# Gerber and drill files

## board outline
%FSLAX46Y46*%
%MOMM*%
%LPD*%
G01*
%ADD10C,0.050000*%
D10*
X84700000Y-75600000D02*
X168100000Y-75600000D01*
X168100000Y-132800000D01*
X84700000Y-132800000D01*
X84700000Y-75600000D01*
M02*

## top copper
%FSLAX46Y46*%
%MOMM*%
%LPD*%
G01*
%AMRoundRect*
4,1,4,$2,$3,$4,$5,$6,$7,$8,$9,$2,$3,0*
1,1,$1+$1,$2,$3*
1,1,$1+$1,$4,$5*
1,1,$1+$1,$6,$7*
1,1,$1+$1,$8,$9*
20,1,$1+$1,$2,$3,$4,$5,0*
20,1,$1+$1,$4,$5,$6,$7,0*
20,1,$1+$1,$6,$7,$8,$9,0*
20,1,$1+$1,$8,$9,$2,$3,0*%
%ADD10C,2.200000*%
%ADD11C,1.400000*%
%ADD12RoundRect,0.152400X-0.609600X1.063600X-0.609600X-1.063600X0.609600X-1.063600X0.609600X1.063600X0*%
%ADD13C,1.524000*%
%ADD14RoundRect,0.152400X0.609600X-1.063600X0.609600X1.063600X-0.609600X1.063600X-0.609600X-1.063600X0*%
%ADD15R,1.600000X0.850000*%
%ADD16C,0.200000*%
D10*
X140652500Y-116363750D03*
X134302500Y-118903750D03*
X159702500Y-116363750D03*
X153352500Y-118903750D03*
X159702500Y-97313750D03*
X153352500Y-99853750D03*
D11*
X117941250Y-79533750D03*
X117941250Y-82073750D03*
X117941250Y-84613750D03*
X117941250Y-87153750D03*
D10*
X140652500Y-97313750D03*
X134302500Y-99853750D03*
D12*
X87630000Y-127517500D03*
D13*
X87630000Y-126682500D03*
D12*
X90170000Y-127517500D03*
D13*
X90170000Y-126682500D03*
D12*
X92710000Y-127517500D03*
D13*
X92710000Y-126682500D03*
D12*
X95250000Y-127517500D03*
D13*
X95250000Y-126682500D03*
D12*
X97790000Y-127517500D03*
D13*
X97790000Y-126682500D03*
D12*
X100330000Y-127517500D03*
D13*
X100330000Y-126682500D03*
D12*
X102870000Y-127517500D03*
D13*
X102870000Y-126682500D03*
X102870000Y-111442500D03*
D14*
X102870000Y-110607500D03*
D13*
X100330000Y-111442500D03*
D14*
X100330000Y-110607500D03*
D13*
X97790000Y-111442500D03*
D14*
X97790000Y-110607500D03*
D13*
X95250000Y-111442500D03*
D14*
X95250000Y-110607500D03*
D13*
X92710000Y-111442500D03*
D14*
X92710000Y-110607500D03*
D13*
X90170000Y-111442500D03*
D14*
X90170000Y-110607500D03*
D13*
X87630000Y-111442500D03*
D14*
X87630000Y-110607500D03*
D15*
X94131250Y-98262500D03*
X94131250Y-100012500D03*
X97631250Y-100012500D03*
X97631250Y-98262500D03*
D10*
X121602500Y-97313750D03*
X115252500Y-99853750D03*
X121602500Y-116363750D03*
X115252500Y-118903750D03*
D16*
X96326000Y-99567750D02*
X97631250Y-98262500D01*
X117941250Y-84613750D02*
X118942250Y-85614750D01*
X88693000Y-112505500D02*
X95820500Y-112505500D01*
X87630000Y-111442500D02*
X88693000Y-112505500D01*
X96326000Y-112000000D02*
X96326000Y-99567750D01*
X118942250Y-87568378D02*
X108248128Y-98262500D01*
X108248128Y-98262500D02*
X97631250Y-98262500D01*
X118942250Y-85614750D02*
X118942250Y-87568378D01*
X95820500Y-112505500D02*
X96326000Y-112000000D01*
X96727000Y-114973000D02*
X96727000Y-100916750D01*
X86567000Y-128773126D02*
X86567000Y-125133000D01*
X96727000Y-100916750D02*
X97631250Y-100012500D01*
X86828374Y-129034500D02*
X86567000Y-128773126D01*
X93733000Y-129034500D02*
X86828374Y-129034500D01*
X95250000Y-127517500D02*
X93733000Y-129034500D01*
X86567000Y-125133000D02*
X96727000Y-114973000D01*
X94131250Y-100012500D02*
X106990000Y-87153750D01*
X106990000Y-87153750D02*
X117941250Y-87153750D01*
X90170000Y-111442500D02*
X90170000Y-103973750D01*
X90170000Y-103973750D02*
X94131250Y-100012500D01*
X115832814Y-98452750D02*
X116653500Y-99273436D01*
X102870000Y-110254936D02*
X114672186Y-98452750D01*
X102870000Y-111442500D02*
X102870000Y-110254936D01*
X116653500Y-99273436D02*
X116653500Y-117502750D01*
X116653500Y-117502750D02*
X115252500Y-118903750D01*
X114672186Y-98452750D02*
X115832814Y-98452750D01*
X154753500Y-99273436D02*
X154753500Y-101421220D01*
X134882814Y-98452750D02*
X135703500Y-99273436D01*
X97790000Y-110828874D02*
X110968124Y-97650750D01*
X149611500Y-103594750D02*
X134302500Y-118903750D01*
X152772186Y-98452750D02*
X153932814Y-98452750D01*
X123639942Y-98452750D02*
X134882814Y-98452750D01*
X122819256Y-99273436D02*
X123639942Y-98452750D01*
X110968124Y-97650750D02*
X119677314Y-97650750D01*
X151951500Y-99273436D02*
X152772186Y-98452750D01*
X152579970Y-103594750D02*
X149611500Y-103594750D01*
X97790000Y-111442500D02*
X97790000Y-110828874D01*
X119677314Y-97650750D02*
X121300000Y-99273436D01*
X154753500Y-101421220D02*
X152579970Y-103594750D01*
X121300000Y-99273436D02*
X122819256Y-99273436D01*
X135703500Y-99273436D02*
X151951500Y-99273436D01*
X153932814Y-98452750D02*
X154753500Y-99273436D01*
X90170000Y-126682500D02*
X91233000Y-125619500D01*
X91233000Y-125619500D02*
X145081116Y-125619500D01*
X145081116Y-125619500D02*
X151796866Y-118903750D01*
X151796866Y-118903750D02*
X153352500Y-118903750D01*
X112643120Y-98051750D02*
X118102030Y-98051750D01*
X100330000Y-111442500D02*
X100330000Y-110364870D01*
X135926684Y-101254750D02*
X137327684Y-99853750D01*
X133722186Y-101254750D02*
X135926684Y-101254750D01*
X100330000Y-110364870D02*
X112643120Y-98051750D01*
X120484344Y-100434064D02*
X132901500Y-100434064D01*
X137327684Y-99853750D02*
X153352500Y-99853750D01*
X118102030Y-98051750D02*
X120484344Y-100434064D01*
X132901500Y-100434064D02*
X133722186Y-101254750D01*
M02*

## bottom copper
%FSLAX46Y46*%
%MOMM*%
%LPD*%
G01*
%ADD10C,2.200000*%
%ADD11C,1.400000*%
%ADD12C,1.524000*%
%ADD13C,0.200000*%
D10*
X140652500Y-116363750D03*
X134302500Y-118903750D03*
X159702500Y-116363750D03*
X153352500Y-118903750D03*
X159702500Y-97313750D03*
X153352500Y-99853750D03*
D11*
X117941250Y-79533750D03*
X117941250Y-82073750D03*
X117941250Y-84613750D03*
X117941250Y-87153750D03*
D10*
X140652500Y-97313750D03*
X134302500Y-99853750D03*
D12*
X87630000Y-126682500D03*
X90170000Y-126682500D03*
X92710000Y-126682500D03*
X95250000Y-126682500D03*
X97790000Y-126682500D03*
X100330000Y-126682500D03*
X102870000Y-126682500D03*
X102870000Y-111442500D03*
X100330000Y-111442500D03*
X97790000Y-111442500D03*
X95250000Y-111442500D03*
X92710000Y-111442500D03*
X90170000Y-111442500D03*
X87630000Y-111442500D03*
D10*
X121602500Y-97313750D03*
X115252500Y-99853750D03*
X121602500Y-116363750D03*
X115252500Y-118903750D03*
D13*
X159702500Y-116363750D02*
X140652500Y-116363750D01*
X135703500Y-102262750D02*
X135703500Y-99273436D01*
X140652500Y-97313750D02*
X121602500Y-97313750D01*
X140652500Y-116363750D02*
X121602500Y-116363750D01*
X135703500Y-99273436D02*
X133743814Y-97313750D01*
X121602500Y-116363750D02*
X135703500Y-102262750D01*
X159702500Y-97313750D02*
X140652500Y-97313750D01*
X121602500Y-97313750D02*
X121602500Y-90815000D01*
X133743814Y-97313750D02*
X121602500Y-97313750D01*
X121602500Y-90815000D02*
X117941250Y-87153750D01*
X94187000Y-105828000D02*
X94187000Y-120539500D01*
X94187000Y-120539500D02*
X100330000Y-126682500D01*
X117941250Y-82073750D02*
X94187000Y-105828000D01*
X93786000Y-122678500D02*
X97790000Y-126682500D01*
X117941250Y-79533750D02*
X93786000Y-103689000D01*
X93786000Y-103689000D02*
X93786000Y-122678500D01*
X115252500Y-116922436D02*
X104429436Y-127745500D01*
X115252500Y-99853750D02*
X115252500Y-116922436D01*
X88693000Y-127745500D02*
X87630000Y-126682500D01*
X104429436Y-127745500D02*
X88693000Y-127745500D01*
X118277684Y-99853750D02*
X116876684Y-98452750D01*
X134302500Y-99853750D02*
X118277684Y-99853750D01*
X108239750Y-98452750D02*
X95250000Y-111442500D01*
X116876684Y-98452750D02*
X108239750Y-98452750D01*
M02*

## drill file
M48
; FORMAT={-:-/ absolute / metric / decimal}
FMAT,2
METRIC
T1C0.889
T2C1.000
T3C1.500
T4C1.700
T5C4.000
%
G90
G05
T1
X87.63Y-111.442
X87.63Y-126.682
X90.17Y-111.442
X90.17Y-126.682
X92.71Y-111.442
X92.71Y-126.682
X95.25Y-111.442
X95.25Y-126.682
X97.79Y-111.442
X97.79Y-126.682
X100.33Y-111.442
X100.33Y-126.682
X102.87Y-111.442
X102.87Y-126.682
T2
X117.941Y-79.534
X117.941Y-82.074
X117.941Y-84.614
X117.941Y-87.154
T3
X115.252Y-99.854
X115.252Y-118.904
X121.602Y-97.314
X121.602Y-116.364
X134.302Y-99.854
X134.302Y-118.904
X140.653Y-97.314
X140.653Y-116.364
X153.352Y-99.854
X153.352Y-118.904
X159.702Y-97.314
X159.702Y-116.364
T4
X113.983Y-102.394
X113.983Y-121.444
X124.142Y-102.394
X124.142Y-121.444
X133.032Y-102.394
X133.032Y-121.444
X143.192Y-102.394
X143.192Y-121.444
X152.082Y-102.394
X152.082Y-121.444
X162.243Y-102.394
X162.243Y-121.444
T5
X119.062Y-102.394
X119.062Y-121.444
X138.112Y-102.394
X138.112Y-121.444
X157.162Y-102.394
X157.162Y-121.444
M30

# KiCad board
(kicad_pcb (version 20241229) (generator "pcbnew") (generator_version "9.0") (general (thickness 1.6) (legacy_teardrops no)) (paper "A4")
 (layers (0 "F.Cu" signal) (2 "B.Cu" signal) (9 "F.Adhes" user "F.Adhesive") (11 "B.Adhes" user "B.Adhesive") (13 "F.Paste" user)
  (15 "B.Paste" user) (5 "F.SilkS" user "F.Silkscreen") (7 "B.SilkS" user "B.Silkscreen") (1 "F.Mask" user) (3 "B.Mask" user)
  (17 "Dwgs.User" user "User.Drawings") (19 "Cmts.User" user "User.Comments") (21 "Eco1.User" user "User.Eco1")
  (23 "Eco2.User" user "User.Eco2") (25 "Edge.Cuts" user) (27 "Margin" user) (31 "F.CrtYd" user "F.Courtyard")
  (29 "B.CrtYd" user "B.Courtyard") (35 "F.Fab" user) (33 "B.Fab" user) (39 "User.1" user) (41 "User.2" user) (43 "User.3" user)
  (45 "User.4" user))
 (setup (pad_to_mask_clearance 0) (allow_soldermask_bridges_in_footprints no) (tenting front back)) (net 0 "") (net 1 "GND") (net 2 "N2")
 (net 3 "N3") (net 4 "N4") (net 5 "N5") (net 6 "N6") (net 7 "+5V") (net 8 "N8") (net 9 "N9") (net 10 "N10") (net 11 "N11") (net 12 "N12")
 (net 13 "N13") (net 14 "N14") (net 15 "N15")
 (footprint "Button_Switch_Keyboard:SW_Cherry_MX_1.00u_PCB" (layer "F.Cu") (at 140.6525 116.36375)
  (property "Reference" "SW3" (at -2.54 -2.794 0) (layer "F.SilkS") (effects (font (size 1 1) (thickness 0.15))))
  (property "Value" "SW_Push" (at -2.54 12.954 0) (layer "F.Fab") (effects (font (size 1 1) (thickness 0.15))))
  (pad "" np_thru_hole circle (at -7.62 5.08) (size 1.7 1.7) (drill 1.7) (layers "*.Cu" "*.Mask"))
  (pad "" np_thru_hole circle (at -2.54 5.08) (size 4 4) (drill 4) (layers "*.Cu" "*.Mask"))
  (pad "" np_thru_hole circle (at 2.54 5.08) (size 1.7 1.7) (drill 1.7) (layers "*.Cu" "*.Mask"))
  (pad "1" thru_hole circle (at 0 0) (size 2.2 2.2) (drill 1.5) (layers "*.Cu" "*.Mask") (remove_unused_layers no) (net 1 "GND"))
  (pad "2" thru_hole circle (at -6.35 2.54) (size 2.2 2.2) (drill 1.5) (layers "*.Cu" "*.Mask") (remove_unused_layers no) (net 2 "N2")))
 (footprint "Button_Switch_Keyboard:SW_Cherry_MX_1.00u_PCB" (layer "F.Cu") (at 159.7025 116.36375)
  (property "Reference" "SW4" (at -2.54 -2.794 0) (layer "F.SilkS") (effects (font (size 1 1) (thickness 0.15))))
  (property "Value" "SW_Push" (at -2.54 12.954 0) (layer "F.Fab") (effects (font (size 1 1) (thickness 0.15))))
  (pad "" np_thru_hole circle (at -7.62 5.08) (size 1.7 1.7) (drill 1.7) (layers "*.Cu" "*.Mask"))
  (pad "" np_thru_hole circle (at -2.54 5.08) (size 4 4) (drill 4) (layers "*.Cu" "*.Mask"))
  (pad "" np_thru_hole circle (at 2.54 5.08) (size 1.7 1.7) (drill 1.7) (layers "*.Cu" "*.Mask"))
  (pad "1" thru_hole circle (at 0 0) (size 2.2 2.2) (drill 1.5) (layers "*.Cu" "*.Mask") (remove_unused_layers no) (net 1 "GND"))
  (pad "2" thru_hole circle (at -6.35 2.54) (size 2.2 2.2) (drill 1.5) (layers "*.Cu" "*.Mask") (remove_unused_layers no) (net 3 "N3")))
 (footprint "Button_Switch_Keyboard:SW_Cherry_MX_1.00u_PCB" (layer "F.Cu") (at 159.7025 97.31375)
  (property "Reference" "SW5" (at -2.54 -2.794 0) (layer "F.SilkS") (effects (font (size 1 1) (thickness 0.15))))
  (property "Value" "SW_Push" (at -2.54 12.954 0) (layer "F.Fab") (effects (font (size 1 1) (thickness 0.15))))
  (pad "" np_thru_hole circle (at -7.62 5.08) (size 1.7 1.7) (drill 1.7) (layers "*.Cu" "*.Mask"))
  (pad "" np_thru_hole circle (at -2.54 5.08) (size 4 4) (drill 4) (layers "*.Cu" "*.Mask"))
  (pad "" np_thru_hole circle (at 2.54 5.08) (size 1.7 1.7) (drill 1.7) (layers "*.Cu" "*.Mask"))
  (pad "1" thru_hole circle (at 0 0) (size 2.2 2.2) (drill 1.5) (layers "*.Cu" "*.Mask") (remove_unused_layers no) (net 1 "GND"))
  (pad "2" thru_hole circle (at -6.35 2.54) (size 2.2 2.2) (drill 1.5) (layers "*.Cu" "*.Mask") (remove_unused_layers no) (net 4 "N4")))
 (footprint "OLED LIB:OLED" (layer "F.Cu") (at 117.94125 83.34375 -90)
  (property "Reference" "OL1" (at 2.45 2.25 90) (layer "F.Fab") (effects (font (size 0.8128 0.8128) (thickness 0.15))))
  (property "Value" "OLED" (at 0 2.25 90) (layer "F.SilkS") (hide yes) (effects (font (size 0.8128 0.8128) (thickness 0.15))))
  (pad "1" thru_hole circle (at -3.81 0 270) (size 1.4 1.4) (drill 1) (layers "*.Cu" "*.Mask") (remove_unused_layers no) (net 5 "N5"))
  (pad "2" thru_hole circle (at -1.27 0 270) (size 1.4 1.4) (drill 1) (layers "*.Cu" "*.Mask") (remove_unused_layers no) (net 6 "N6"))
  (pad "3" thru_hole circle (at 1.27 0 270) (size 1.4 1.4) (drill 1) (layers "*.Cu" "*.Mask") (remove_unused_layers no) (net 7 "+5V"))
  (pad "4" thru_hole circle (at 3.81 0 270) (size 1.4 1.4) (drill 1) (layers "*.Cu" "*.Mask") (remove_unused_layers no) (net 1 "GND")))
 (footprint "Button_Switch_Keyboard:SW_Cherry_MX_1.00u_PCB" (layer "F.Cu") (at 140.6525 97.31375)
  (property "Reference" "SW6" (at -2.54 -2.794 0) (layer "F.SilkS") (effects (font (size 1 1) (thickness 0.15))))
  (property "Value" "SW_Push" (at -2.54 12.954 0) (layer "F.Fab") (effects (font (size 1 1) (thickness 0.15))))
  (pad "" np_thru_hole circle (at -7.62 5.08) (size 1.7 1.7) (drill 1.7) (layers "*.Cu" "*.Mask"))
  (pad "" np_thru_hole circle (at -2.54 5.08) (size 4 4) (drill 4) (layers "*.Cu" "*.Mask"))
  (pad "" np_thru_hole circle (at 2.54 5.08) (size 1.7 1.7) (drill 1.7) (layers "*.Cu" "*.Mask"))
  (pad "1" thru_hole circle (at 0 0) (size 2.2 2.2) (drill 1.5) (layers "*.Cu" "*.Mask") (remove_unused_layers no) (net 1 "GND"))
  (pad "2" thru_hole circle (at -6.35 2.54) (size 2.2 2.2) (drill 1.5) (layers "*.Cu" "*.Mask") (remove_unused_layers no) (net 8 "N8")))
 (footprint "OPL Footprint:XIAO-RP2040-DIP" (layer "F.Cu") (at 95.25 119.0625 90)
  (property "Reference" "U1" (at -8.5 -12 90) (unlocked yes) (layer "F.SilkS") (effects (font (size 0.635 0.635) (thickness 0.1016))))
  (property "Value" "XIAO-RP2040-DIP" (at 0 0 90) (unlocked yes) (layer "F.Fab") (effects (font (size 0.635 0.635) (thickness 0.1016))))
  (pad "1" smd roundrect (at -8.455 -7.62 270) (size 2.432 1.524) (layers "F.Cu" "F.Mask") (roundrect_rratio 0.1) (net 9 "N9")
   (thermal_bridge_angle 45))
  (pad "1" thru_hole circle (at -7.62 -7.62 270) (size 1.524 1.524) (drill 0.889) (layers "*.Cu" "*.Mask") (remove_unused_layers no)
   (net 9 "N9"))
  (pad "2" smd roundrect (at -8.455 -5.08 270) (size 2.432 1.524) (layers "F.Cu" "F.Mask") (roundrect_rratio 0.1) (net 3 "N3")
   (thermal_bridge_angle 45))
  (pad "2" thru_hole circle (at -7.62 -5.08 270) (size 1.524 1.524) (drill 0.889) (layers "*.Cu" "*.Mask") (remove_unused_layers no)
   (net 3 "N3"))
  (pad "3" smd roundrect (at -8.455 -2.54 270) (size 2.432 1.524) (layers "F.Cu" "F.Mask") (roundrect_rratio 0.1) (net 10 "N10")
   (thermal_bridge_angle 45))
  (pad "3" thru_hole circle (at -7.62 -2.54 270) (size 1.524 1.524) (drill 0.889) (layers "*.Cu" "*.Mask") (remove_unused_layers no)
   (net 10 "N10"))
  (pad "4" smd roundrect (at -8.455 0 270) (size 2.432 1.524) (layers "F.Cu" "F.Mask") (roundrect_rratio 0.1) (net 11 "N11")
   (thermal_bridge_angle 45))
  (pad "4" thru_hole circle (at -7.62 0 270) (size 1.524 1.524) (drill 0.889) (layers "*.Cu" "*.Mask") (remove_unused_layers no)
   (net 11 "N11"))
  (pad "5" smd roundrect (at -8.455 2.54 270) (size 2.432 1.524) (layers "F.Cu" "F.Mask") (roundrect_rratio 0.1) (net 5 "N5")
   (thermal_bridge_angle 45))
  (pad "5" thru_hole circle (at -7.62 2.54 270) (size 1.524 1.524) (drill 0.889) (layers "*.Cu" "*.Mask") (remove_unused_layers no)
   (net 5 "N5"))
  (pad "6" smd roundrect (at -8.455 5.08 270) (size 2.432 1.524) (layers "F.Cu" "F.Mask") (roundrect_rratio 0.1) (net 6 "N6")
   (thermal_bridge_angle 45))
  (pad "6" thru_hole circle (at -7.62 5.08 270) (size 1.524 1.524) (drill 0.889) (layers "*.Cu" "*.Mask") (remove_unused_layers no)
   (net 6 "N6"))
  (pad "7" smd roundrect (at -8.455 7.62 270) (size 2.432 1.524) (layers "F.Cu" "F.Mask") (roundrect_rratio 0.1) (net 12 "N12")
   (thermal_bridge_angle 45))
  (pad "7" thru_hole circle (at -7.62 7.62 270) (size 1.524 1.524) (drill 0.889) (layers "*.Cu" "*.Mask") (remove_unused_layers no)
   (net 12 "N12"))
  (pad "8" thru_hole circle (at 7.62 7.62 90) (size 1.524 1.524) (drill 0.889) (layers "*.Cu" "*.Mask") (remove_unused_layers no)
   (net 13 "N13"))
  (pad "8" smd roundrect (at 8.455 7.62 90) (size 2.432 1.524) (layers "F.Cu" "F.Mask") (roundrect_rratio 0.1) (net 13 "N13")
   (thermal_bridge_angle 45))
  (pad "9" thru_hole circle (at 7.62 5.08 90) (size 1.524 1.524) (drill 0.889) (layers "*.Cu" "*.Mask") (remove_unused_layers no)
   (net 4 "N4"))
  (pad "9" smd roundrect (at 8.455 5.08 90) (size 2.432 1.524) (layers "F.Cu" "F.Mask") (roundrect_rratio 0.1) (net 4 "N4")
   (thermal_bridge_angle 45))
  (pad "10" thru_hole circle (at 7.62 2.54 90) (size 1.524 1.524) (drill 0.889) (layers "*.Cu" "*.Mask") (remove_unused_layers no)
   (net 2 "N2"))
  (pad "10" smd roundrect (at 8.455 2.54 90) (size 2.432 1.524) (layers "F.Cu" "F.Mask") (roundrect_rratio 0.1) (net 2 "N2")
   (thermal_bridge_angle 45))
  (pad "11" thru_hole circle (at 7.62 0 90) (size 1.524 1.524) (drill 0.889) (layers "*.Cu" "*.Mask") (remove_unused_layers no) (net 8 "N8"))
  (pad "11" smd roundrect (at 8.455 0 90) (size 2.432 1.524) (layers "F.Cu" "F.Mask") (roundrect_rratio 0.1) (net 8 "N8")
   (thermal_bridge_angle 45))
  (pad "12" thru_hole circle (at 7.62 -2.54 90) (size 1.524 1.524) (drill 0.889) (layers "*.Cu" "*.Mask") (remove_unused_layers no)
   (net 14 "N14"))
  (pad "12" smd roundrect (at 8.455 -2.54 90) (size 2.432 1.524) (layers "F.Cu" "F.Mask") (roundrect_rratio 0.1) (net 14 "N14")
   (thermal_bridge_angle 45))
  (pad "13" thru_hole circle (at 7.62 -5.08 90) (size 1.524 1.524) (drill 0.889) (layers "*.Cu" "*.Mask") (remove_unused_layers no)
   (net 1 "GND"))
  (pad "13" smd roundrect (at 8.455 -5.08 90) (size 2.432 1.524) (layers "F.Cu" "F.Mask") (roundrect_rratio 0.1) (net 1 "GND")
   (thermal_bridge_angle 45))
  (pad "14" thru_hole circle (at 7.62 -7.62 90) (size 1.524 1.524) (drill 0.889) (layers "*.Cu" "*.Mask") (remove_unused_layers no)
   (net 7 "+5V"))
  (pad "14" smd roundrect (at 8.455 -7.62 90) (size 2.432 1.524) (layers "F.Cu" "F.Mask") (roundrect_rratio 0.1) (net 7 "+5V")
   (thermal_bridge_angle 45)))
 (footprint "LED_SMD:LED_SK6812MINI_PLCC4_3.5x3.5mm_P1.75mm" (layer "F.Cu") (at 95.88125 99.1375)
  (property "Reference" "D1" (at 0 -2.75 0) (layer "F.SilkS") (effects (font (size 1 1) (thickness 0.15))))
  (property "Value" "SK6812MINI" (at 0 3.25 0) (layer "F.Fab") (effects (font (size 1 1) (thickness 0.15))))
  (pad "1" smd rect (at -1.75 -0.875) (size 1.6 0.85) (layers "F.Cu" "F.Mask" "F.Paste") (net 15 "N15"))
  (pad "2" smd rect (at -1.75 0.875) (size 1.6 0.85) (layers "F.Cu" "F.Mask" "F.Paste") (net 1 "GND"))
  (pad "3" smd rect (at 1.75 0.875) (size 1.6 0.85) (layers "F.Cu" "F.Mask" "F.Paste") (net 11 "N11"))
  (pad "4" smd rect (at 1.75 -0.875) (size 1.6 0.85) (layers "F.Cu" "F.Mask" "F.Paste") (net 7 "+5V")))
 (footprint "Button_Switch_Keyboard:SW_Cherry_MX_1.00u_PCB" (layer "F.Cu") (at 121.6025 97.31375)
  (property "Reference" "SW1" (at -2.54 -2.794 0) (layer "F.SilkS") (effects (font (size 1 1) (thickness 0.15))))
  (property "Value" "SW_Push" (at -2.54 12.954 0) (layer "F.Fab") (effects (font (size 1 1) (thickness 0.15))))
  (pad "" np_thru_hole circle (at -7.62 5.08) (size 1.7 1.7) (drill 1.7) (layers "*.Cu" "*.Mask"))
  (pad "" np_thru_hole circle (at -2.54 5.08) (size 4 4) (drill 4) (layers "*.Cu" "*.Mask"))
  (pad "" np_thru_hole circle (at 2.54 5.08) (size 1.7 1.7) (drill 1.7) (layers "*.Cu" "*.Mask"))
  (pad "1" thru_hole circle (at 0 0) (size 2.2 2.2) (drill 1.5) (layers "*.Cu" "*.Mask") (remove_unused_layers no) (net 1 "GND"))
  (pad "2" thru_hole circle (at -6.35 2.54) (size 2.2 2.2) (drill 1.5) (layers "*.Cu" "*.Mask") (remove_unused_layers no) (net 9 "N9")))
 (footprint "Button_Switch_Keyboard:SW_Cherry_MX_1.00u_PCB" (layer "F.Cu") (at 121.6025 116.36375)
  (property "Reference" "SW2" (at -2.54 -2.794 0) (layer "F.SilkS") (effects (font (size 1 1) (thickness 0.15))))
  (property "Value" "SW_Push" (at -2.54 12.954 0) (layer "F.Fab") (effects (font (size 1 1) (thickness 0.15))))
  (pad "" np_thru_hole circle (at -7.62 5.08) (size 1.7 1.7) (drill 1.7) (layers "*.Cu" "*.Mask"))
  (pad "" np_thru_hole circle (at -2.54 5.08) (size 4 4) (drill 4) (layers "*.Cu" "*.Mask"))
  (pad "" np_thru_hole circle (at 2.54 5.08) (size 1.7 1.7) (drill 1.7) (layers "*.Cu" "*.Mask"))
  (pad "1" thru_hole circle (at 0 0) (size 2.2 2.2) (drill 1.5) (layers "*.Cu" "*.Mask") (remove_unused_layers no) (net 1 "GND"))
  (pad "2" thru_hole circle (at -6.35 2.54) (size 2.2 2.2) (drill 1.5) (layers "*.Cu" "*.Mask") (remove_unused_layers no) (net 13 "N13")))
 (gr_rect (start 84.7 75.6) (end 168.1 132.8) (stroke (width 0.05) (type default)) (fill no) (layer "Edge.Cuts"))
 (segment (start 96.326 99.56775) (end 97.63125 98.2625) (width 0.2) (layer "F.Cu") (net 7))
 (segment (start 117.94125 84.61375) (end 118.94225 85.61475) (width 0.2) (layer "F.Cu") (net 7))
 (segment (start 88.693 112.5055) (end 95.8205 112.5055) (width 0.2) (layer "F.Cu") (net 7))
 (segment (start 87.63 111.4425) (end 88.693 112.5055) (width 0.2) (layer "F.Cu") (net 7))
 (segment (start 96.326 112) (end 96.326 99.56775) (width 0.2) (layer "F.Cu") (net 7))
 (segment (start 118.94225 87.568378) (end 108.248128 98.2625) (width 0.2) (layer "F.Cu") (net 7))
 (segment (start 108.248128 98.2625) (end 97.63125 98.2625) (width 0.2) (layer "F.Cu") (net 7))
 (segment (start 118.94225 85.61475) (end 118.94225 87.568378) (width 0.2) (layer "F.Cu") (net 7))
 (segment (start 95.8205 112.5055) (end 96.326 112) (width 0.2) (layer "F.Cu") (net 7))
 (segment (start 96.727 114.973) (end 96.727 100.91675) (width 0.2) (layer "F.Cu") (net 11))
 (segment (start 86.567 128.773126) (end 86.567 125.133) (width 0.2) (layer "F.Cu") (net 11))
 (segment (start 96.727 100.91675) (end 97.63125 100.0125) (width 0.2) (layer "F.Cu") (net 11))
 (segment (start 86.828374 129.0345) (end 86.567 128.773126) (width 0.2) (layer "F.Cu") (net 11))
 (segment (start 93.733 129.0345) (end 86.828374 129.0345) (width 0.2) (layer "F.Cu") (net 11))
 (segment (start 95.25 127.5175) (end 93.733 129.0345) (width 0.2) (layer "F.Cu") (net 11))
 (segment (start 86.567 125.133) (end 96.727 114.973) (width 0.2) (layer "F.Cu") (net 11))
 (segment (start 94.13125 100.0125) (end 106.99 87.15375) (width 0.2) (layer "F.Cu") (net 1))
 (segment (start 106.99 87.15375) (end 117.94125 87.15375) (width 0.2) (layer "F.Cu") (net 1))
 (segment (start 90.17 111.4425) (end 90.17 103.97375) (width 0.2) (layer "F.Cu") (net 1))
 (segment (start 90.17 103.97375) (end 94.13125 100.0125) (width 0.2) (layer "F.Cu") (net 1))
 (segment (start 159.7025 116.36375) (end 140.6525 116.36375) (width 0.2) (layer "B.Cu") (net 1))
 (segment (start 135.7035 102.26275) (end 135.7035 99.273436) (width 0.2) (layer "B.Cu") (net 1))
 (segment (start 140.6525 97.31375) (end 121.6025 97.31375) (width 0.2) (layer "B.Cu") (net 1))
 (segment (start 140.6525 116.36375) (end 121.6025 116.36375) (width 0.2) (layer "B.Cu") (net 1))
 (segment (start 135.7035 99.273436) (end 133.743814 97.31375) (width 0.2) (layer "B.Cu") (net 1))
 (segment (start 121.6025 116.36375) (end 135.7035 102.26275) (width 0.2) (layer "B.Cu") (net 1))
 (segment (start 159.7025 97.31375) (end 140.6525 97.31375) (width 0.2) (layer "B.Cu") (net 1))
 (segment (start 121.6025 97.31375) (end 121.6025 90.815) (width 0.2) (layer "B.Cu") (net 1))
 (segment (start 133.743814 97.31375) (end 121.6025 97.31375) (width 0.2) (layer "B.Cu") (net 1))
 (segment (start 121.6025 90.815) (end 117.94125 87.15375) (width 0.2) (layer "B.Cu") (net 1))
 (segment (start 94.187 105.828) (end 94.187 120.5395) (width 0.2) (layer "B.Cu") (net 6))
 (segment (start 94.187 120.5395) (end 100.33 126.6825) (width 0.2) (layer "B.Cu") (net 6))
 (segment (start 117.94125 82.07375) (end 94.187 105.828) (width 0.2) (layer "B.Cu") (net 6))
 (segment (start 93.786 122.6785) (end 97.79 126.6825) (width 0.2) (layer "B.Cu") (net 5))
 (segment (start 117.94125 79.53375) (end 93.786 103.689) (width 0.2) (layer "B.Cu") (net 5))
 (segment (start 93.786 103.689) (end 93.786 122.6785) (width 0.2) (layer "B.Cu") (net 5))
 (segment (start 115.2525 116.922436) (end 104.429436 127.7455) (width 0.2) (layer "B.Cu") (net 9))
 (segment (start 115.2525 99.85375) (end 115.2525 116.922436) (width 0.2) (layer "B.Cu") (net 9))
 (segment (start 88.693 127.7455) (end 87.63 126.6825) (width 0.2) (layer "B.Cu") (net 9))
 (segment (start 104.429436 127.7455) (end 88.693 127.7455) (width 0.2) (layer "B.Cu") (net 9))
 (segment (start 115.832814 98.45275) (end 116.6535 99.273436) (width 0.2) (layer "F.Cu") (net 13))
 (segment (start 102.87 110.254936) (end 114.672186 98.45275) (width 0.2) (layer "F.Cu") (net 13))
 (segment (start 102.87 111.4425) (end 102.87 110.254936) (width 0.2) (layer "F.Cu") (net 13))
 (segment (start 116.6535 99.273436) (end 116.6535 117.50275) (width 0.2) (layer "F.Cu") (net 13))
 (segment (start 116.6535 117.50275) (end 115.2525 118.90375) (width 0.2) (layer "F.Cu") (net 13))
 (segment (start 114.672186 98.45275) (end 115.832814 98.45275) (width 0.2) (layer "F.Cu") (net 13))
 (segment (start 154.7535 99.273436) (end 154.7535 101.42122) (width 0.2) (layer "F.Cu") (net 2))
 (segment (start 134.882814 98.45275) (end 135.7035 99.273436) (width 0.2) (layer "F.Cu") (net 2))
 (segment (start 97.79 110.828874) (end 110.968124 97.65075) (width 0.2) (layer "F.Cu") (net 2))
 (segment (start 149.6115 103.59475) (end 134.3025 118.90375) (width 0.2) (layer "F.Cu") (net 2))
 (segment (start 152.772186 98.45275) (end 153.932814 98.45275) (width 0.2) (layer "F.Cu") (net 2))
 (segment (start 123.639942 98.45275) (end 134.882814 98.45275) (width 0.2) (layer "F.Cu") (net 2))
 (segment (start 122.819256 99.273436) (end 123.639942 98.45275) (width 0.2) (layer "F.Cu") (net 2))
 (segment (start 110.968124 97.65075) (end 119.677314 97.65075) (width 0.2) (layer "F.Cu") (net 2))
 (segment (start 151.9515 99.273436) (end 152.772186 98.45275) (width 0.2) (layer "F.Cu") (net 2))
 (segment (start 152.57997 103.59475) (end 149.6115 103.59475) (width 0.2) (layer "F.Cu") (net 2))
 (segment (start 97.79 111.4425) (end 97.79 110.828874) (width 0.2) (layer "F.Cu") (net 2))
 (segment (start 119.677314 97.65075) (end 121.3 99.273436) (width 0.2) (layer "F.Cu") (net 2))
 (segment (start 154.7535 101.42122) (end 152.57997 103.59475) (width 0.2) (layer "F.Cu") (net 2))
 (segment (start 121.3 99.273436) (end 122.819256 99.273436) (width 0.2) (layer "F.Cu") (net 2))
 (segment (start 135.7035 99.273436) (end 151.9515 99.273436) (width 0.2) (layer "F.Cu") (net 2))
 (segment (start 153.932814 98.45275) (end 154.7535 99.273436) (width 0.2) (layer "F.Cu") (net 2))
 (segment (start 90.17 126.6825) (end 91.233 125.6195) (width 0.2) (layer "F.Cu") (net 3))
 (segment (start 91.233 125.6195) (end 145.081116 125.6195) (width 0.2) (layer "F.Cu") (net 3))
 (segment (start 145.081116 125.6195) (end 151.796866 118.90375) (width 0.2) (layer "F.Cu") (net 3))
 (segment (start 151.796866 118.90375) (end 153.3525 118.90375) (width 0.2) (layer "F.Cu") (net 3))
 (segment (start 112.64312 98.05175) (end 118.10203 98.05175) (width 0.2) (layer "F.Cu") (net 4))
 (segment (start 100.33 111.4425) (end 100.33 110.36487) (width 0.2) (layer "F.Cu") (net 4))
 (segment (start 135.926684 101.25475) (end 137.327684 99.85375) (width 0.2) (layer "F.Cu") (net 4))
 (segment (start 133.722186 101.25475) (end 135.926684 101.25475) (width 0.2) (layer "F.Cu") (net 4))
 (segment (start 100.33 110.36487) (end 112.64312 98.05175) (width 0.2) (layer "F.Cu") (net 4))
 (segment (start 120.484344 100.434064) (end 132.9015 100.434064) (width 0.2) (layer "F.Cu") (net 4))
 (segment (start 137.327684 99.85375) (end 153.3525 99.85375) (width 0.2) (layer "F.Cu") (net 4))
 (segment (start 118.10203 98.05175) (end 120.484344 100.434064) (width 0.2) (layer "F.Cu") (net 4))
 (segment (start 132.9015 100.434064) (end 133.722186 101.25475) (width 0.2) (layer "F.Cu") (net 4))
 (segment (start 118.277684 99.85375) (end 116.876684 98.45275) (width 0.2) (layer "B.Cu") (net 8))
 (segment (start 134.3025 99.85375) (end 118.277684 99.85375) (width 0.2) (layer "B.Cu") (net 8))
 (segment (start 108.23975 98.45275) (end 95.25 111.4425) (width 0.2) (layer "B.Cu") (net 8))
 (segment (start 116.876684 98.45275) (end 108.23975 98.45275) (width 0.2) (layer "B.Cu") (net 8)))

